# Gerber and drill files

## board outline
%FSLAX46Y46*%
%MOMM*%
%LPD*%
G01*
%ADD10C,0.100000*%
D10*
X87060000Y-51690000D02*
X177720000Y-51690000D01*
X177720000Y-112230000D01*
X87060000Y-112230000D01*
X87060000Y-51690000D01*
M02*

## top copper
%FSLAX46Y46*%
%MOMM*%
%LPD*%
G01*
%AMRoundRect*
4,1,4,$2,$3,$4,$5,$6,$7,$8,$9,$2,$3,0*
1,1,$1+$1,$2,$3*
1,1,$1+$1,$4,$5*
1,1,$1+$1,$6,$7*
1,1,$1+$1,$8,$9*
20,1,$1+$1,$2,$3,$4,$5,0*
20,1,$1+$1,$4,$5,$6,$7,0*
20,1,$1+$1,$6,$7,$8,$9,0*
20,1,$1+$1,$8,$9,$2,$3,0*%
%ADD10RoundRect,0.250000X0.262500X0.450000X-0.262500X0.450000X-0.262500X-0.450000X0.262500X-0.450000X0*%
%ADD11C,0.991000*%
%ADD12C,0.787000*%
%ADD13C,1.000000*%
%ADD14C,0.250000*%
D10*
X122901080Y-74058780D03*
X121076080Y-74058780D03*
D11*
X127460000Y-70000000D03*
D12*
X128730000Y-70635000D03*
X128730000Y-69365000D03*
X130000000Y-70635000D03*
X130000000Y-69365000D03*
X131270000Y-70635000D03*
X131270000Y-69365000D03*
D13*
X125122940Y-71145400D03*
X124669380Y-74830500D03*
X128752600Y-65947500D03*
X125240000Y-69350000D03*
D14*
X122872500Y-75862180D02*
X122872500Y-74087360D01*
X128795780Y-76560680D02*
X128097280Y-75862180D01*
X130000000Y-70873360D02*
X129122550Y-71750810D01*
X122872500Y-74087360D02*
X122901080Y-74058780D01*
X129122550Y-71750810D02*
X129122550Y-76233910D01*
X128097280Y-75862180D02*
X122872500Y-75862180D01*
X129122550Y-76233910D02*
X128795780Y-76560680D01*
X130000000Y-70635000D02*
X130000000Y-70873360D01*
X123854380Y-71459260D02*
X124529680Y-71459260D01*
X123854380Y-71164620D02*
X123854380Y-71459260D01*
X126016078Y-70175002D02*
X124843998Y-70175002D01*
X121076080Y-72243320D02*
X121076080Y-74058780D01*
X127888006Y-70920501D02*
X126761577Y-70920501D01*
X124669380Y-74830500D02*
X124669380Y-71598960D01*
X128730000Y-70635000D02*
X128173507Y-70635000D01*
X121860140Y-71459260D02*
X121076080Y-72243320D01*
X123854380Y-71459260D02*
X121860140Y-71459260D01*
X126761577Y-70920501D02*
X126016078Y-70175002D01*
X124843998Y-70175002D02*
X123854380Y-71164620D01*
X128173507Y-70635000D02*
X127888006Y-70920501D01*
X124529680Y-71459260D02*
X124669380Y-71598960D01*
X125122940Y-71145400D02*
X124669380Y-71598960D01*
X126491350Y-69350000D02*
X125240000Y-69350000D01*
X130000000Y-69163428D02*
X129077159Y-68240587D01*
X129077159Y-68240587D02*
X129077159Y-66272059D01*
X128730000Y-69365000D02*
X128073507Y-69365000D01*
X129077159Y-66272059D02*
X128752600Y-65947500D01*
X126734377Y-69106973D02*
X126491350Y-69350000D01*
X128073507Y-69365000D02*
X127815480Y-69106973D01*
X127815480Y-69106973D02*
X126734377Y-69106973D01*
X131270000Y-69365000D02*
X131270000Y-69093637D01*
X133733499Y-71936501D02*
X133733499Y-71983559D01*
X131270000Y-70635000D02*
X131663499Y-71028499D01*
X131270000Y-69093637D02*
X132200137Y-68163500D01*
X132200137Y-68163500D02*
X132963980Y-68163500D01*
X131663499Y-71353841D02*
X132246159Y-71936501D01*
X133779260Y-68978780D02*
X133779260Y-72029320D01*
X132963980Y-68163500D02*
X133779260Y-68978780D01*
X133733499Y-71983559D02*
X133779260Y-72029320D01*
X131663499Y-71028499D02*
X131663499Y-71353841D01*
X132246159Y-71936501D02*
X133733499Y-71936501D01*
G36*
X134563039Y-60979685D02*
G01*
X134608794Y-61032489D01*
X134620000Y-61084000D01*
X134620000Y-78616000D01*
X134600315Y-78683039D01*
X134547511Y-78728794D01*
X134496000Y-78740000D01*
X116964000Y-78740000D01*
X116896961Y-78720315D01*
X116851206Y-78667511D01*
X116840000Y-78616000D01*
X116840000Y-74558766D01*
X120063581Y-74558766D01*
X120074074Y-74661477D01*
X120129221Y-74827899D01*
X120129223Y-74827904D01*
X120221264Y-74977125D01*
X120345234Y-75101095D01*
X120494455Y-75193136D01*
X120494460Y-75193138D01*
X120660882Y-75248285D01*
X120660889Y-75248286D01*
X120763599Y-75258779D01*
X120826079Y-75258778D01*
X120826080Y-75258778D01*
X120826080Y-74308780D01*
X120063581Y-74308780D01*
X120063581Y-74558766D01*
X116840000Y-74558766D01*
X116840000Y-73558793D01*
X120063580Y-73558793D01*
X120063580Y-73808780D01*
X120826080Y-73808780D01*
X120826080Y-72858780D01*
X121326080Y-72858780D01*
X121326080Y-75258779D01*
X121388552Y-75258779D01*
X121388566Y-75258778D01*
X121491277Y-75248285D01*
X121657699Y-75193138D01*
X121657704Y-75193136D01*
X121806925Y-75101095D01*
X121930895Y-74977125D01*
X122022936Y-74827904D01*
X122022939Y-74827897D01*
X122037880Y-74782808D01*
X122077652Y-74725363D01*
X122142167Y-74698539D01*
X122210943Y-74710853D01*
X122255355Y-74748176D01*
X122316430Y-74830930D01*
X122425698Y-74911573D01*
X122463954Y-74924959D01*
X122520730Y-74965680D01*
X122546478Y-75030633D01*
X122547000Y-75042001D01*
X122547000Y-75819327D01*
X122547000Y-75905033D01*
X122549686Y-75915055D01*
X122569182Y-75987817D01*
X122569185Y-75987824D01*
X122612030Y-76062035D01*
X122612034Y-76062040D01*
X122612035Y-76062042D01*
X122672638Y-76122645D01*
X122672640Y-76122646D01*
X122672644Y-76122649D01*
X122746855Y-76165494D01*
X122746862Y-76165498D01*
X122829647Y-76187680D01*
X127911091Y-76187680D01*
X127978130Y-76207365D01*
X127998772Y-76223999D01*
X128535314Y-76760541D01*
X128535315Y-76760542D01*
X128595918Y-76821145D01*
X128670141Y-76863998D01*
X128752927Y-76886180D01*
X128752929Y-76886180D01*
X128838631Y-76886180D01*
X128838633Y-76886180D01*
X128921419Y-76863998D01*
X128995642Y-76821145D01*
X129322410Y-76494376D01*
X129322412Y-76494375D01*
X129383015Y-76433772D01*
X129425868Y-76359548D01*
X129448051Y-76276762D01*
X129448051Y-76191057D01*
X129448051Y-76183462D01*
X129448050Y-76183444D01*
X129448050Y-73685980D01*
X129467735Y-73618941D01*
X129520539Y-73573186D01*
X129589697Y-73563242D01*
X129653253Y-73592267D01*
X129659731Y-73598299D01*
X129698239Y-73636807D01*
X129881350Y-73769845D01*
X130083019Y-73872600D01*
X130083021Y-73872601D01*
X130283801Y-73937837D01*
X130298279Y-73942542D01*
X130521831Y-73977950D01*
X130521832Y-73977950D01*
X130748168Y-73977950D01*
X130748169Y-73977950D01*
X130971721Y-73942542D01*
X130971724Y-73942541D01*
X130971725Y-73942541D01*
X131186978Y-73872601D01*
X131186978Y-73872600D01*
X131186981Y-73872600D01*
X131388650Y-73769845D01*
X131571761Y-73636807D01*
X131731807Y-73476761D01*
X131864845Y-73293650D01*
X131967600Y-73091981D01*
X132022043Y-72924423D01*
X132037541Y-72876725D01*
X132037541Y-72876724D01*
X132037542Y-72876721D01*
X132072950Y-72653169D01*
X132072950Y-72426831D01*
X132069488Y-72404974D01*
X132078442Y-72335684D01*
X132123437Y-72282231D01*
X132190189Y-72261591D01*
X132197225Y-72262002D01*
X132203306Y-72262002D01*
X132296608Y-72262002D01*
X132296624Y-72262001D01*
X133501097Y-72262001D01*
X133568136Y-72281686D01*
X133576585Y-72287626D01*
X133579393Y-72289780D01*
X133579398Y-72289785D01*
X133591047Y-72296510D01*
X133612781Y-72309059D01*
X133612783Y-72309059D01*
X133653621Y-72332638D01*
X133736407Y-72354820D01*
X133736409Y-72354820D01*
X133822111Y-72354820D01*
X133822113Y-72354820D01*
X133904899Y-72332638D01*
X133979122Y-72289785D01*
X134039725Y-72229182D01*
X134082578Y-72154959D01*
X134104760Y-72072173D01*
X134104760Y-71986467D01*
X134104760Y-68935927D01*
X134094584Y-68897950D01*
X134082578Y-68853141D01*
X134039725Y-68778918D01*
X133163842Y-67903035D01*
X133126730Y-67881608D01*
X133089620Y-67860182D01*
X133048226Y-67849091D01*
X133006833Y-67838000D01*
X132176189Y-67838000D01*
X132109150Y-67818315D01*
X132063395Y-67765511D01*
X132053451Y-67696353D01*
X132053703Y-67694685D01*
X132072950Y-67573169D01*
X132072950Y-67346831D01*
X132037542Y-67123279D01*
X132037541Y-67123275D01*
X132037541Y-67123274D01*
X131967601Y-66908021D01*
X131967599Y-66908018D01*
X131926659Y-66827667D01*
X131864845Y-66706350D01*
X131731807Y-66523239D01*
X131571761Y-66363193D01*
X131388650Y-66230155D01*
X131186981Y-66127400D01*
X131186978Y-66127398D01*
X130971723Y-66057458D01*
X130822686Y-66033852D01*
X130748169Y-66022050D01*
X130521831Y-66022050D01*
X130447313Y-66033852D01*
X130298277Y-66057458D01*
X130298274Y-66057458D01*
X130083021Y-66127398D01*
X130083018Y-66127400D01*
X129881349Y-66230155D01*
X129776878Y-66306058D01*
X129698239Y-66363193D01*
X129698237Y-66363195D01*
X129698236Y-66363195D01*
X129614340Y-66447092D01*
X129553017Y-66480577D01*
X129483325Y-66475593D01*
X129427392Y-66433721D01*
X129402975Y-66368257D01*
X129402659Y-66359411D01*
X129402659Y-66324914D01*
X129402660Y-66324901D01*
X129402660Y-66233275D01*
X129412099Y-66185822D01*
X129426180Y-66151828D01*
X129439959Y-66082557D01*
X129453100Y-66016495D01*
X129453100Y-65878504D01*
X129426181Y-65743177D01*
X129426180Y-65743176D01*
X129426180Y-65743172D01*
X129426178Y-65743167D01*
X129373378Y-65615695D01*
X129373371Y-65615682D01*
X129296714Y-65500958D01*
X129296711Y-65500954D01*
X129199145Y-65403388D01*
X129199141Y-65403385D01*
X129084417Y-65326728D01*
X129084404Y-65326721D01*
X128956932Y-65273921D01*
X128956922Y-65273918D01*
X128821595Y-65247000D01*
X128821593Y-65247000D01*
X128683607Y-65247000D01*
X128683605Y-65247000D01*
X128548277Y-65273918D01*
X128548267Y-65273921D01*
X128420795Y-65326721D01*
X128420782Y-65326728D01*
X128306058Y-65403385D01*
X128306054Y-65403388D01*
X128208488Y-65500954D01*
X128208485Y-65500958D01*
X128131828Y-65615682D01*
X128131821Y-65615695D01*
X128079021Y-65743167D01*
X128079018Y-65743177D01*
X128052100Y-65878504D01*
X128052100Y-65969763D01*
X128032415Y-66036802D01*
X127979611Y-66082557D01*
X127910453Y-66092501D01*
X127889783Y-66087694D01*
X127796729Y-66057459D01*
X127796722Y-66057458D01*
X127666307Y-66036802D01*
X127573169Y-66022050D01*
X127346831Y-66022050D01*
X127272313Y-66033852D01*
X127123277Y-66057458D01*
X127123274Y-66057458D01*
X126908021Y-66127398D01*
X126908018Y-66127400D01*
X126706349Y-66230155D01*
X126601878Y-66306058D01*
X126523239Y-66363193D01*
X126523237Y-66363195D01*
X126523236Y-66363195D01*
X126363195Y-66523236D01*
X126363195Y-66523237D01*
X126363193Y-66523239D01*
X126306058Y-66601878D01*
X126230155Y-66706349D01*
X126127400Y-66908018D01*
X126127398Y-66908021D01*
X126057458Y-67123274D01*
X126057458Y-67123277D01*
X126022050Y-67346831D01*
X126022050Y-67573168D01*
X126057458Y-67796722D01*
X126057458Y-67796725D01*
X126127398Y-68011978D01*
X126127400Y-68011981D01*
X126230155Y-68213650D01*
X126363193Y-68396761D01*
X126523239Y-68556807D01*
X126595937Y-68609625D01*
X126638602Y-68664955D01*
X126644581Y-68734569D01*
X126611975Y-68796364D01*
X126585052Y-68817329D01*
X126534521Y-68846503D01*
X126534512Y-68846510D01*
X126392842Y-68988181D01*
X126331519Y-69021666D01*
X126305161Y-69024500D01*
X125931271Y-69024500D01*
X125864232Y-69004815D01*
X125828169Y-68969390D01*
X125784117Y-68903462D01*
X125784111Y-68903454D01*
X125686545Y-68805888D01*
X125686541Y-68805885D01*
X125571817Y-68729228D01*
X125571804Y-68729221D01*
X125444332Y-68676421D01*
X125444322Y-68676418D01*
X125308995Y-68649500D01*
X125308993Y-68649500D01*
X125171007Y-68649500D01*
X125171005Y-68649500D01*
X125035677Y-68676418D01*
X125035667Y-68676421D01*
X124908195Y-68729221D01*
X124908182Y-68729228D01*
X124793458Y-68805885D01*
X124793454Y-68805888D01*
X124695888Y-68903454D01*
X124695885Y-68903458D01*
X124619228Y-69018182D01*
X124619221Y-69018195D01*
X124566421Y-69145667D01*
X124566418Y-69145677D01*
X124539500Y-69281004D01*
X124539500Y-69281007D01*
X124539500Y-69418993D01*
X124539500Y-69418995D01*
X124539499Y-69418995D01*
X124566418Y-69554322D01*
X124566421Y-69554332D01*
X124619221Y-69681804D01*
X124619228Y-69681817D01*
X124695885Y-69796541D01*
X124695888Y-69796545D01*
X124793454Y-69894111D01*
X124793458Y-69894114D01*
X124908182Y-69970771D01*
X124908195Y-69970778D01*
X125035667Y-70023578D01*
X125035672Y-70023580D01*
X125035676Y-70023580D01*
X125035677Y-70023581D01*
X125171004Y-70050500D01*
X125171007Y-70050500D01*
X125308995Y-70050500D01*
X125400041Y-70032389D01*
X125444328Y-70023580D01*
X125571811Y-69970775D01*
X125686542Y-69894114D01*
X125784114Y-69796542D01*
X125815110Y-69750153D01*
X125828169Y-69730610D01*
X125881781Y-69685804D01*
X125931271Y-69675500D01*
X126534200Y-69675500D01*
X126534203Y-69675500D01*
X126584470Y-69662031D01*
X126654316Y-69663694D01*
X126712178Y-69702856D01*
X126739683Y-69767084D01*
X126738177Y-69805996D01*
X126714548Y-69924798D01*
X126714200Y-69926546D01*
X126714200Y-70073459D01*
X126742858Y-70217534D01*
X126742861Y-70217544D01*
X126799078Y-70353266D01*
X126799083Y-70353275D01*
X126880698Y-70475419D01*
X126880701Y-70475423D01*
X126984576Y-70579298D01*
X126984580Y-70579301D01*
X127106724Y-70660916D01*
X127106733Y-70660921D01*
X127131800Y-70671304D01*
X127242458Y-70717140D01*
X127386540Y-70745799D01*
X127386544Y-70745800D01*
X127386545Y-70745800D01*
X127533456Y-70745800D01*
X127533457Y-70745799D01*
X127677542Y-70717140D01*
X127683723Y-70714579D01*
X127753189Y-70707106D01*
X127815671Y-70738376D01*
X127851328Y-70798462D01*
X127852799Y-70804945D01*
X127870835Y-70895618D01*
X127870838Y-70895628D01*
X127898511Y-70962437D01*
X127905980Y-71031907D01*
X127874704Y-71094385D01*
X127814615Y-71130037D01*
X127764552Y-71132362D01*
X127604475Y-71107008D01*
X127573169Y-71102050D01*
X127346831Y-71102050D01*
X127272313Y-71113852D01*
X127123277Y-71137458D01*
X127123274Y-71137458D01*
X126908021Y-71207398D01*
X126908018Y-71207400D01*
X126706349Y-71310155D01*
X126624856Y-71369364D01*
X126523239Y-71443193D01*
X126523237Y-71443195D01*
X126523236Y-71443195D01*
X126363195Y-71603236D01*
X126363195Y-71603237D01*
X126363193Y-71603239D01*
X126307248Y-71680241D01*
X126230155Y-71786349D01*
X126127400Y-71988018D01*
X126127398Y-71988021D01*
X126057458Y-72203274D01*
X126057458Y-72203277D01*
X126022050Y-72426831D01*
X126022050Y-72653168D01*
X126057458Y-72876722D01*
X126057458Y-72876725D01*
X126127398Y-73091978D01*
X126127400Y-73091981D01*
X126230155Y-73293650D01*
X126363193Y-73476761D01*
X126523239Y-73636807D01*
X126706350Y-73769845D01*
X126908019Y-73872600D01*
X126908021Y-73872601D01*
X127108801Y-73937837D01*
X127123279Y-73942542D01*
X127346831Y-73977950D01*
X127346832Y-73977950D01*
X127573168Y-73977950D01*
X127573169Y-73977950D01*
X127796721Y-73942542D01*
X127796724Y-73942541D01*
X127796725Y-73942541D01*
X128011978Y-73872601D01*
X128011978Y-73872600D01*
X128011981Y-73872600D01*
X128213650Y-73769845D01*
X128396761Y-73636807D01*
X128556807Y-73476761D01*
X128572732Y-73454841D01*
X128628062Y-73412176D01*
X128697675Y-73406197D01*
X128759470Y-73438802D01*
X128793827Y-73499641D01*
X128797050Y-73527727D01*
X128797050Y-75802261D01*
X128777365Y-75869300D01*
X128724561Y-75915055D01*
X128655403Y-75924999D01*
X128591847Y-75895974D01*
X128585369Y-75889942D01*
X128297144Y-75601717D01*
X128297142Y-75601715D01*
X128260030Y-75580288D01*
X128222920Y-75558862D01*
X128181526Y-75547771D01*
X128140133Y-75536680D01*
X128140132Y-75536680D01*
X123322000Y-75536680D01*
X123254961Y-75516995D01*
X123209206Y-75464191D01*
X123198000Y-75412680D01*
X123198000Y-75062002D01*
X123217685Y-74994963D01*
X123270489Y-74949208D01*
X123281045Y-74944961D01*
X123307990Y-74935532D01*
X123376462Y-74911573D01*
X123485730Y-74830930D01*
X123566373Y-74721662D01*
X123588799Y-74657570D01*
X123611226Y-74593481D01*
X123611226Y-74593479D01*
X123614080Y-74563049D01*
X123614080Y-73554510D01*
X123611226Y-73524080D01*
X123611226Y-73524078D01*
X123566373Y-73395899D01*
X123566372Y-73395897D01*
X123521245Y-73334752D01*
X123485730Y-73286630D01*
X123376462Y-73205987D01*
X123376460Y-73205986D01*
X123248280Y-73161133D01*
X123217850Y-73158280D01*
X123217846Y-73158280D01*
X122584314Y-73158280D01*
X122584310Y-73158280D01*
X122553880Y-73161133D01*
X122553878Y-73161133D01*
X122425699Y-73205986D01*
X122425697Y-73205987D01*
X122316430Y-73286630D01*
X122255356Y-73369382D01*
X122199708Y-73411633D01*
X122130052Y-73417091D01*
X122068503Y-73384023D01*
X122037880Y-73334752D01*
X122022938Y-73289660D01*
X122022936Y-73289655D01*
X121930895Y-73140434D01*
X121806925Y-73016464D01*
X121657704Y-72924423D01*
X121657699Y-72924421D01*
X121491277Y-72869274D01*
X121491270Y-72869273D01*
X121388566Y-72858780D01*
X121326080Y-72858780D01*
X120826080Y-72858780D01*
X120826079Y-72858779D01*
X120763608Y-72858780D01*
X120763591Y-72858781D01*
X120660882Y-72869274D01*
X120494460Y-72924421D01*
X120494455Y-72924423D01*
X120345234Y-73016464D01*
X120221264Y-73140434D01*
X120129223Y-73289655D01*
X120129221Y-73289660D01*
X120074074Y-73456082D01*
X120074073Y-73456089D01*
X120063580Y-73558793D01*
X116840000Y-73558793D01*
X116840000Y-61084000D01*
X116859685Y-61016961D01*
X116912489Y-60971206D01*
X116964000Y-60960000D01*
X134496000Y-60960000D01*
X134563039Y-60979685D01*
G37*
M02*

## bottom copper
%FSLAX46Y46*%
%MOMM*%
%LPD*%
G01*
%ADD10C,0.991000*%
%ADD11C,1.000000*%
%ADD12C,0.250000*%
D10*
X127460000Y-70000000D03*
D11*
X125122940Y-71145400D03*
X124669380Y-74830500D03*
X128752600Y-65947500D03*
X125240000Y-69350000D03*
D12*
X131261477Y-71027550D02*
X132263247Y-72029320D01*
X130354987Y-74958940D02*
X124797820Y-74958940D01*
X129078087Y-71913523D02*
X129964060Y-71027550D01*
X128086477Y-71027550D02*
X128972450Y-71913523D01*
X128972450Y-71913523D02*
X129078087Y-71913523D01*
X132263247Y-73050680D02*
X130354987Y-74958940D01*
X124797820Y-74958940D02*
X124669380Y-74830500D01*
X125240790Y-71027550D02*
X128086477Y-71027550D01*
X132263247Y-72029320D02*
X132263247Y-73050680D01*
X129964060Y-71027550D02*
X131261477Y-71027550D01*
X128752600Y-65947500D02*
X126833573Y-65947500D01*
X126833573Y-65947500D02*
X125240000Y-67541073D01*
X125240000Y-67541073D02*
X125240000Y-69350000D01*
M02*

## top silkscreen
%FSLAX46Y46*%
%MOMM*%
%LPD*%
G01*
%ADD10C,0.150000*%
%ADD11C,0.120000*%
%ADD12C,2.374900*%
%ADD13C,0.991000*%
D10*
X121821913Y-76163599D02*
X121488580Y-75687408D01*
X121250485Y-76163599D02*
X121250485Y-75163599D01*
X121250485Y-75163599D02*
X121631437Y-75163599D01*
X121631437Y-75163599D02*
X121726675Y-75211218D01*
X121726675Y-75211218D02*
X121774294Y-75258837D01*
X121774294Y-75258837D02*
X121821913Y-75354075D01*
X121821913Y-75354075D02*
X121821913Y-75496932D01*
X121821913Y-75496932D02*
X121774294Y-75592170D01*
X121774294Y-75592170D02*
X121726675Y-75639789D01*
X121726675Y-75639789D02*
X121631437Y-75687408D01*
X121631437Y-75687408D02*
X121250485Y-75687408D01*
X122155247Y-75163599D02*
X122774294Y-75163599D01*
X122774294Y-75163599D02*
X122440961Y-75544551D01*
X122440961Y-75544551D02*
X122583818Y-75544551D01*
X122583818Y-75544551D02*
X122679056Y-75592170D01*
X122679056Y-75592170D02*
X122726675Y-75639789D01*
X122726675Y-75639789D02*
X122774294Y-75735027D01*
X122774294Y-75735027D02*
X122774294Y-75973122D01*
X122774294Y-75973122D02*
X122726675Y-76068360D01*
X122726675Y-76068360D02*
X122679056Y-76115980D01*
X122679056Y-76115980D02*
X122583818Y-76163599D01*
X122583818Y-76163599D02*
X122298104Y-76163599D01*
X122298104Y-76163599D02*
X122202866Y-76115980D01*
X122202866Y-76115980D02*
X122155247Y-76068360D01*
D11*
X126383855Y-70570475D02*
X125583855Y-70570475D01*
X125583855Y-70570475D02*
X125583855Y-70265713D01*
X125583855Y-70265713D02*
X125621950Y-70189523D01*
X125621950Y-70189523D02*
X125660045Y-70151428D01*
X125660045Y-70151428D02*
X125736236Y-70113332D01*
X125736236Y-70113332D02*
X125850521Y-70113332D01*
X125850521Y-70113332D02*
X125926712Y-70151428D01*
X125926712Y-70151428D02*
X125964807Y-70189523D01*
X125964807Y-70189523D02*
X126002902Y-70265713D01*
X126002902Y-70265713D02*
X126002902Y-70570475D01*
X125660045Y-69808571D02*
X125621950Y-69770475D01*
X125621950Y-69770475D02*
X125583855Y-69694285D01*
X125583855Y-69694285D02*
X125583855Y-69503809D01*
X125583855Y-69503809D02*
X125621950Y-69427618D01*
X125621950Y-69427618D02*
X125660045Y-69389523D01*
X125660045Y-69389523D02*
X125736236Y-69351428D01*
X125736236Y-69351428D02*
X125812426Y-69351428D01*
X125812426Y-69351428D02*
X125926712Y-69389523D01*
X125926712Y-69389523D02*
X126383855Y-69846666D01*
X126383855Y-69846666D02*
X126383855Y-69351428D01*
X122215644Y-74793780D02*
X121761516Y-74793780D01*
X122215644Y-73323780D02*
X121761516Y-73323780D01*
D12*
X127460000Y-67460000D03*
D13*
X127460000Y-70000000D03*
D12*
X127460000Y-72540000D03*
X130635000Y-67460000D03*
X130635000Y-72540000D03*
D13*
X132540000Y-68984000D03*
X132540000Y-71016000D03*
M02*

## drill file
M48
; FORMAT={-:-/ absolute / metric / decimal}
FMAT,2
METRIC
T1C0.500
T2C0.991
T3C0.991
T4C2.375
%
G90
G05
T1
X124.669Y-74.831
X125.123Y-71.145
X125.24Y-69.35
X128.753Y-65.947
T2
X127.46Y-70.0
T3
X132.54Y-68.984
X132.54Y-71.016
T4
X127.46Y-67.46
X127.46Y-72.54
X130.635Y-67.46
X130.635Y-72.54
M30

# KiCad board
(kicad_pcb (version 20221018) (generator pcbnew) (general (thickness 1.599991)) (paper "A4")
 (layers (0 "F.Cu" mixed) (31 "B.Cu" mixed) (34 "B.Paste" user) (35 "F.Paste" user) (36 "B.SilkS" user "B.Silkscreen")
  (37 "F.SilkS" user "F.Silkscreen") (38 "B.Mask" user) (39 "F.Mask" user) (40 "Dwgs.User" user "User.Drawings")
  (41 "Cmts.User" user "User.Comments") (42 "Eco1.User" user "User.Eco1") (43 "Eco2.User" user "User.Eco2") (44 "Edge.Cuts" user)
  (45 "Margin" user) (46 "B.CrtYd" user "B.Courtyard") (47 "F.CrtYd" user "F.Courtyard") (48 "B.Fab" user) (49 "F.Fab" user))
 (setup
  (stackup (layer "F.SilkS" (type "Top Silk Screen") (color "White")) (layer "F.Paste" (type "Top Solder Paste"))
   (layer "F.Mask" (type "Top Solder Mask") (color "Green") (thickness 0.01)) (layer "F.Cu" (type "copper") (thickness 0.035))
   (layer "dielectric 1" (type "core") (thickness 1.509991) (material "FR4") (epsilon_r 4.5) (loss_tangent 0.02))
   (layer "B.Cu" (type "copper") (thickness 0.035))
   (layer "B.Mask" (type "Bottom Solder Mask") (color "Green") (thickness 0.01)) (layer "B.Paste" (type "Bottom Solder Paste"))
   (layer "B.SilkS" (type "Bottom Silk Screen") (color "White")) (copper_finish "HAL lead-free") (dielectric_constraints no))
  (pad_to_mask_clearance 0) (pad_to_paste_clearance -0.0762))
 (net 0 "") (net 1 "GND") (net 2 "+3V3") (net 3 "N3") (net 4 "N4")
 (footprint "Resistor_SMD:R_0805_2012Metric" (layer "F.Cu") (at 121.98858 74.05878 180)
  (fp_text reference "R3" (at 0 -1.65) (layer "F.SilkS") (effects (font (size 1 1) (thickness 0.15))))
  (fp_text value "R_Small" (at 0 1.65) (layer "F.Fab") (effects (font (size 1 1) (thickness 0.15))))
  (fp_line (start -0.227064 -0.735) (end 0.227064 -0.735) (stroke (width 0.12) (type solid)) (layer "F.SilkS"))
  (fp_line (start -0.227064 0.735) (end 0.227064 0.735) (stroke (width 0.12) (type solid)) (layer "F.SilkS"))
  (pad "1" smd roundrect (at -0.9125 0 180) (size 1.025 1.4) (layers "F.Cu" "F.Paste" "F.Mask") (roundrect_rratio 0.243902) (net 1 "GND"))
  (pad "2" smd roundrect (at 0.9125 0 180) (size 1.025 1.4) (layers "F.Cu" "F.Paste" "F.Mask") (roundrect_rratio 0.243902) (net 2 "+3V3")))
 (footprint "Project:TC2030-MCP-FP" (layer "F.Cu") (at 130 70)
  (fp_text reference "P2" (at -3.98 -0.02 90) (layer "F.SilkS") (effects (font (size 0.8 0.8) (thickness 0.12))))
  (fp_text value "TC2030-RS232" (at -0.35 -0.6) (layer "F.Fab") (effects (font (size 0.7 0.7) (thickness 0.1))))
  (pad "" np_thru_hole circle (at -2.54 -2.54) (size 2.3749 2.3749) (drill 2.3749) (layers "*.Cu" "*.Mask" "F.SilkS"))
  (pad "" np_thru_hole circle (at -2.54 0) (size 0.991 0.991) (drill 0.9906) (layers "*.Cu" "*.Mask" "F.SilkS"))
  (pad "" np_thru_hole circle (at -2.54 2.54) (size 2.3749 2.3749) (drill 2.3749) (layers "*.Cu" "*.Mask" "F.SilkS"))
  (pad "" np_thru_hole circle (at 0.635 -2.54) (size 2.3749 2.3749) (drill 2.3749) (layers "*.Cu" "*.Mask" "F.SilkS"))
  (pad "" np_thru_hole circle (at 0.635 2.54) (size 2.3749 2.3749) (drill 2.3749) (layers "*.Cu" "*.Mask" "F.SilkS"))
  (pad "" np_thru_hole circle (at 2.54 -1.016) (size 0.991 0.991) (drill 0.991) (layers "*.Cu" "*.Mask" "F.SilkS"))
  (pad "" np_thru_hole circle (at 2.54 1.016) (size 0.991 0.991) (drill 0.991) (layers "*.Cu" "*.Mask" "F.SilkS"))
  (pad "1" connect circle (at -1.27 0.635) (size 0.787 0.787) (layers "F.Cu" "F.Mask") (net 2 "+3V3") (clearance 0.4826))
  (pad "2" connect circle (at -1.27 -0.635) (size 0.787 0.787) (layers "F.Cu" "F.Mask") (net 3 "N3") (clearance 0.4826))
  (pad "3" connect circle (at 0 0.635) (size 0.787 0.787) (layers "F.Cu" "F.Mask") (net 1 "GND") (clearance 0.4191))
  (pad "4" connect circle (at 0 -0.635) (size 0.787 0.787) (layers "F.Cu" "F.Mask") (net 3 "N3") (clearance 0.4191))
  (pad "5" connect circle (at 1.27 0.635) (size 0.787 0.787) (layers "F.Cu" "F.Mask") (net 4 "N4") (clearance 0.4191))
  (pad "6" connect circle (at 1.27 -0.635 90) (size 0.787 0.787) (layers "F.Cu" "F.Mask") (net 4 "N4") (clearance 0.4191)))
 (gr_rect (start 87.06 51.69) (end 177.72 112.23) (stroke (width 0.1) (type solid)) (fill none) (layer "Edge.Cuts"))
 (segment (start 122.8725 75.86218) (end 122.8725 74.08736) (width 0.25) (layer "F.Cu") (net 1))
 (segment (start 128.79578 76.56068) (end 128.09728 75.86218) (width 0.25) (layer "F.Cu") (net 1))
 (segment (start 130 70.87336) (end 129.12255 71.75081) (width 0.25) (layer "F.Cu") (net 1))
 (segment (start 122.8725 74.08736) (end 122.90108 74.05878) (width 0.25) (layer "F.Cu") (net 1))
 (segment (start 129.12255 71.75081) (end 129.12255 76.23391) (width 0.25) (layer "F.Cu") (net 1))
 (segment (start 128.09728 75.86218) (end 122.8725 75.86218) (width 0.25) (layer "F.Cu") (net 1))
 (segment (start 129.12255 76.23391) (end 128.79578 76.56068) (width 0.25) (layer "F.Cu") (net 1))
 (segment (start 130 70.635) (end 130 70.87336) (width 0.25) (layer "F.Cu") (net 1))
 (segment (start 123.85438 71.45926) (end 124.52968 71.45926) (width 0.25) (layer "F.Cu") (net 2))
 (segment (start 123.85438 71.16462) (end 123.85438 71.45926) (width 0.25) (layer "F.Cu") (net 2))
 (segment (start 126.016078 70.175002) (end 124.843998 70.175002) (width 0.25) (layer "F.Cu") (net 2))
 (segment (start 121.07608 72.24332) (end 121.07608 74.05878) (width 0.25) (layer "F.Cu") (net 2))
 (segment (start 127.888006 70.920501) (end 126.761577 70.920501) (width 0.25) (layer "F.Cu") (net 2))
 (segment (start 124.66938 74.8305) (end 124.66938 71.59896) (width 0.25) (layer "F.Cu") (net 2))
 (segment (start 128.73 70.635) (end 128.173507 70.635) (width 0.25) (layer "F.Cu") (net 2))
 (segment (start 121.86014 71.45926) (end 121.07608 72.24332) (width 0.25) (layer "F.Cu") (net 2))
 (segment (start 123.85438 71.45926) (end 121.86014 71.45926) (width 0.25) (layer "F.Cu") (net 2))
 (segment (start 126.761577 70.920501) (end 126.016078 70.175002) (width 0.25) (layer "F.Cu") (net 2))
 (segment (start 124.843998 70.175002) (end 123.85438 71.16462) (width 0.25) (layer "F.Cu") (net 2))
 (segment (start 128.173507 70.635) (end 127.888006 70.920501) (width 0.25) (layer "F.Cu") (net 2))
 (segment (start 124.52968 71.45926) (end 124.66938 71.59896) (width 0.25) (layer "F.Cu") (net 2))
 (segment (start 125.12294 71.1454) (end 124.66938 71.59896) (width 0.25) (layer "F.Cu") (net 2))
 (via (at 125.12294 71.1454) (size 1) (drill 0.5) (layers "F.Cu" "B.Cu") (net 2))
 (via (at 124.66938 74.8305) (size 1) (drill 0.5) (layers "F.Cu" "B.Cu") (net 2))
 (segment (start 131.261477 71.02755) (end 132.263247 72.02932) (width 0.25) (layer "B.Cu") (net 2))
 (segment (start 130.354987 74.95894) (end 124.79782 74.95894) (width 0.25) (layer "B.Cu") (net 2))
 (segment (start 129.078087 71.913523) (end 129.96406 71.02755) (width 0.25) (layer "B.Cu") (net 2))
 (segment (start 128.086477 71.02755) (end 128.97245 71.913523) (width 0.25) (layer "B.Cu") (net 2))
 (segment (start 128.97245 71.913523) (end 129.078087 71.913523) (width 0.25) (layer "B.Cu") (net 2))
 (segment (start 132.263247 73.05068) (end 130.354987 74.95894) (width 0.25) (layer "B.Cu") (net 2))
 (segment (start 124.79782 74.95894) (end 124.66938 74.8305) (width 0.25) (layer "B.Cu") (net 2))
 (segment (start 125.24079 71.02755) (end 128.086477 71.02755) (width 0.25) (layer "B.Cu") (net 2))
 (segment (start 132.263247 72.02932) (end 132.263247 73.05068) (width 0.25) (layer "B.Cu") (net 2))
 (segment (start 129.96406 71.02755) (end 131.261477 71.02755) (width 0.25) (layer "B.Cu") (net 2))
 (segment (start 126.49135 69.35) (end 125.24 69.35) (width 0.25) (layer "F.Cu") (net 3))
 (segment (start 130 69.163428) (end 129.077159 68.240587) (width 0.25) (layer "F.Cu") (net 3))
 (segment (start 129.077159 68.240587) (end 129.077159 66.272059) (width 0.25) (layer "F.Cu") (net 3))
 (segment (start 128.73 69.365) (end 128.073507 69.365) (width 0.25) (layer "F.Cu") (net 3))
 (segment (start 129.077159 66.272059) (end 128.7526 65.9475) (width 0.25) (layer "F.Cu") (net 3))
 (segment (start 126.734377 69.106973) (end 126.49135 69.35) (width 0.25) (layer "F.Cu") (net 3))
 (segment (start 128.073507 69.365) (end 127.81548 69.106973) (width 0.25) (layer "F.Cu") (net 3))
 (segment (start 127.81548 69.106973) (end 126.734377 69.106973) (width 0.25) (layer "F.Cu") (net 3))
 (via (at 128.7526 65.9475) (size 1) (drill 0.5) (layers "F.Cu" "B.Cu") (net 3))
 (via (at 125.24 69.35) (size 1) (drill 0.5) (layers "F.Cu" "B.Cu") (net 3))
 (segment (start 128.7526 65.9475) (end 126.833573 65.9475) (width 0.25) (layer "B.Cu") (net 3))
 (segment (start 126.833573 65.9475) (end 125.24 67.541073) (width 0.25) (layer "B.Cu") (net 3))
 (segment (start 125.24 67.541073) (end 125.24 69.35) (width 0.25) (layer "B.Cu") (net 3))
 (segment (start 131.27 69.365) (end 131.27 69.093637) (width 0.25) (layer "F.Cu") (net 4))
 (segment (start 133.733499 71.936501) (end 133.733499 71.983559) (width 0.25) (layer "F.Cu") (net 4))
 (segment (start 131.27 70.635) (end 131.663499 71.028499) (width 0.25) (layer "F.Cu") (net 4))
 (segment (start 131.27 69.093637) (end 132.200137 68.1635) (width 0.25) (layer "F.Cu") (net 4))
 (segment (start 132.200137 68.1635) (end 132.96398 68.1635) (width 0.25) (layer "F.Cu") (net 4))
 (segment (start 131.663499 71.353841) (end 132.246159 71.936501) (width 0.25) (layer "F.Cu") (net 4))
 (segment (start 133.77926 68.97878) (end 133.77926 72.02932) (width 0.25) (layer "F.Cu") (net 4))
 (segment (start 132.96398 68.1635) (end 133.77926 68.97878) (width 0.25) (layer "F.Cu") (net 4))
 (segment (start 133.733499 71.983559) (end 133.77926 72.02932) (width 0.25) (layer "F.Cu") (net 4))
 (segment (start 131.663499 71.028499) (end 131.663499 71.353841) (width 0.25) (layer "F.Cu") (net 4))
 (segment (start 132.246159 71.936501) (end 133.733499 71.936501) (width 0.25) (layer "F.Cu") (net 4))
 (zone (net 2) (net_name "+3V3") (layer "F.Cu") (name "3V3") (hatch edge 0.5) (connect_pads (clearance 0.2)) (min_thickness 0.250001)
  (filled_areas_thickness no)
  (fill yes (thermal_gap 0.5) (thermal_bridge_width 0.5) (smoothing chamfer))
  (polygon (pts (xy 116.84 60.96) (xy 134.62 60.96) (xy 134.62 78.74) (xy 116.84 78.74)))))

